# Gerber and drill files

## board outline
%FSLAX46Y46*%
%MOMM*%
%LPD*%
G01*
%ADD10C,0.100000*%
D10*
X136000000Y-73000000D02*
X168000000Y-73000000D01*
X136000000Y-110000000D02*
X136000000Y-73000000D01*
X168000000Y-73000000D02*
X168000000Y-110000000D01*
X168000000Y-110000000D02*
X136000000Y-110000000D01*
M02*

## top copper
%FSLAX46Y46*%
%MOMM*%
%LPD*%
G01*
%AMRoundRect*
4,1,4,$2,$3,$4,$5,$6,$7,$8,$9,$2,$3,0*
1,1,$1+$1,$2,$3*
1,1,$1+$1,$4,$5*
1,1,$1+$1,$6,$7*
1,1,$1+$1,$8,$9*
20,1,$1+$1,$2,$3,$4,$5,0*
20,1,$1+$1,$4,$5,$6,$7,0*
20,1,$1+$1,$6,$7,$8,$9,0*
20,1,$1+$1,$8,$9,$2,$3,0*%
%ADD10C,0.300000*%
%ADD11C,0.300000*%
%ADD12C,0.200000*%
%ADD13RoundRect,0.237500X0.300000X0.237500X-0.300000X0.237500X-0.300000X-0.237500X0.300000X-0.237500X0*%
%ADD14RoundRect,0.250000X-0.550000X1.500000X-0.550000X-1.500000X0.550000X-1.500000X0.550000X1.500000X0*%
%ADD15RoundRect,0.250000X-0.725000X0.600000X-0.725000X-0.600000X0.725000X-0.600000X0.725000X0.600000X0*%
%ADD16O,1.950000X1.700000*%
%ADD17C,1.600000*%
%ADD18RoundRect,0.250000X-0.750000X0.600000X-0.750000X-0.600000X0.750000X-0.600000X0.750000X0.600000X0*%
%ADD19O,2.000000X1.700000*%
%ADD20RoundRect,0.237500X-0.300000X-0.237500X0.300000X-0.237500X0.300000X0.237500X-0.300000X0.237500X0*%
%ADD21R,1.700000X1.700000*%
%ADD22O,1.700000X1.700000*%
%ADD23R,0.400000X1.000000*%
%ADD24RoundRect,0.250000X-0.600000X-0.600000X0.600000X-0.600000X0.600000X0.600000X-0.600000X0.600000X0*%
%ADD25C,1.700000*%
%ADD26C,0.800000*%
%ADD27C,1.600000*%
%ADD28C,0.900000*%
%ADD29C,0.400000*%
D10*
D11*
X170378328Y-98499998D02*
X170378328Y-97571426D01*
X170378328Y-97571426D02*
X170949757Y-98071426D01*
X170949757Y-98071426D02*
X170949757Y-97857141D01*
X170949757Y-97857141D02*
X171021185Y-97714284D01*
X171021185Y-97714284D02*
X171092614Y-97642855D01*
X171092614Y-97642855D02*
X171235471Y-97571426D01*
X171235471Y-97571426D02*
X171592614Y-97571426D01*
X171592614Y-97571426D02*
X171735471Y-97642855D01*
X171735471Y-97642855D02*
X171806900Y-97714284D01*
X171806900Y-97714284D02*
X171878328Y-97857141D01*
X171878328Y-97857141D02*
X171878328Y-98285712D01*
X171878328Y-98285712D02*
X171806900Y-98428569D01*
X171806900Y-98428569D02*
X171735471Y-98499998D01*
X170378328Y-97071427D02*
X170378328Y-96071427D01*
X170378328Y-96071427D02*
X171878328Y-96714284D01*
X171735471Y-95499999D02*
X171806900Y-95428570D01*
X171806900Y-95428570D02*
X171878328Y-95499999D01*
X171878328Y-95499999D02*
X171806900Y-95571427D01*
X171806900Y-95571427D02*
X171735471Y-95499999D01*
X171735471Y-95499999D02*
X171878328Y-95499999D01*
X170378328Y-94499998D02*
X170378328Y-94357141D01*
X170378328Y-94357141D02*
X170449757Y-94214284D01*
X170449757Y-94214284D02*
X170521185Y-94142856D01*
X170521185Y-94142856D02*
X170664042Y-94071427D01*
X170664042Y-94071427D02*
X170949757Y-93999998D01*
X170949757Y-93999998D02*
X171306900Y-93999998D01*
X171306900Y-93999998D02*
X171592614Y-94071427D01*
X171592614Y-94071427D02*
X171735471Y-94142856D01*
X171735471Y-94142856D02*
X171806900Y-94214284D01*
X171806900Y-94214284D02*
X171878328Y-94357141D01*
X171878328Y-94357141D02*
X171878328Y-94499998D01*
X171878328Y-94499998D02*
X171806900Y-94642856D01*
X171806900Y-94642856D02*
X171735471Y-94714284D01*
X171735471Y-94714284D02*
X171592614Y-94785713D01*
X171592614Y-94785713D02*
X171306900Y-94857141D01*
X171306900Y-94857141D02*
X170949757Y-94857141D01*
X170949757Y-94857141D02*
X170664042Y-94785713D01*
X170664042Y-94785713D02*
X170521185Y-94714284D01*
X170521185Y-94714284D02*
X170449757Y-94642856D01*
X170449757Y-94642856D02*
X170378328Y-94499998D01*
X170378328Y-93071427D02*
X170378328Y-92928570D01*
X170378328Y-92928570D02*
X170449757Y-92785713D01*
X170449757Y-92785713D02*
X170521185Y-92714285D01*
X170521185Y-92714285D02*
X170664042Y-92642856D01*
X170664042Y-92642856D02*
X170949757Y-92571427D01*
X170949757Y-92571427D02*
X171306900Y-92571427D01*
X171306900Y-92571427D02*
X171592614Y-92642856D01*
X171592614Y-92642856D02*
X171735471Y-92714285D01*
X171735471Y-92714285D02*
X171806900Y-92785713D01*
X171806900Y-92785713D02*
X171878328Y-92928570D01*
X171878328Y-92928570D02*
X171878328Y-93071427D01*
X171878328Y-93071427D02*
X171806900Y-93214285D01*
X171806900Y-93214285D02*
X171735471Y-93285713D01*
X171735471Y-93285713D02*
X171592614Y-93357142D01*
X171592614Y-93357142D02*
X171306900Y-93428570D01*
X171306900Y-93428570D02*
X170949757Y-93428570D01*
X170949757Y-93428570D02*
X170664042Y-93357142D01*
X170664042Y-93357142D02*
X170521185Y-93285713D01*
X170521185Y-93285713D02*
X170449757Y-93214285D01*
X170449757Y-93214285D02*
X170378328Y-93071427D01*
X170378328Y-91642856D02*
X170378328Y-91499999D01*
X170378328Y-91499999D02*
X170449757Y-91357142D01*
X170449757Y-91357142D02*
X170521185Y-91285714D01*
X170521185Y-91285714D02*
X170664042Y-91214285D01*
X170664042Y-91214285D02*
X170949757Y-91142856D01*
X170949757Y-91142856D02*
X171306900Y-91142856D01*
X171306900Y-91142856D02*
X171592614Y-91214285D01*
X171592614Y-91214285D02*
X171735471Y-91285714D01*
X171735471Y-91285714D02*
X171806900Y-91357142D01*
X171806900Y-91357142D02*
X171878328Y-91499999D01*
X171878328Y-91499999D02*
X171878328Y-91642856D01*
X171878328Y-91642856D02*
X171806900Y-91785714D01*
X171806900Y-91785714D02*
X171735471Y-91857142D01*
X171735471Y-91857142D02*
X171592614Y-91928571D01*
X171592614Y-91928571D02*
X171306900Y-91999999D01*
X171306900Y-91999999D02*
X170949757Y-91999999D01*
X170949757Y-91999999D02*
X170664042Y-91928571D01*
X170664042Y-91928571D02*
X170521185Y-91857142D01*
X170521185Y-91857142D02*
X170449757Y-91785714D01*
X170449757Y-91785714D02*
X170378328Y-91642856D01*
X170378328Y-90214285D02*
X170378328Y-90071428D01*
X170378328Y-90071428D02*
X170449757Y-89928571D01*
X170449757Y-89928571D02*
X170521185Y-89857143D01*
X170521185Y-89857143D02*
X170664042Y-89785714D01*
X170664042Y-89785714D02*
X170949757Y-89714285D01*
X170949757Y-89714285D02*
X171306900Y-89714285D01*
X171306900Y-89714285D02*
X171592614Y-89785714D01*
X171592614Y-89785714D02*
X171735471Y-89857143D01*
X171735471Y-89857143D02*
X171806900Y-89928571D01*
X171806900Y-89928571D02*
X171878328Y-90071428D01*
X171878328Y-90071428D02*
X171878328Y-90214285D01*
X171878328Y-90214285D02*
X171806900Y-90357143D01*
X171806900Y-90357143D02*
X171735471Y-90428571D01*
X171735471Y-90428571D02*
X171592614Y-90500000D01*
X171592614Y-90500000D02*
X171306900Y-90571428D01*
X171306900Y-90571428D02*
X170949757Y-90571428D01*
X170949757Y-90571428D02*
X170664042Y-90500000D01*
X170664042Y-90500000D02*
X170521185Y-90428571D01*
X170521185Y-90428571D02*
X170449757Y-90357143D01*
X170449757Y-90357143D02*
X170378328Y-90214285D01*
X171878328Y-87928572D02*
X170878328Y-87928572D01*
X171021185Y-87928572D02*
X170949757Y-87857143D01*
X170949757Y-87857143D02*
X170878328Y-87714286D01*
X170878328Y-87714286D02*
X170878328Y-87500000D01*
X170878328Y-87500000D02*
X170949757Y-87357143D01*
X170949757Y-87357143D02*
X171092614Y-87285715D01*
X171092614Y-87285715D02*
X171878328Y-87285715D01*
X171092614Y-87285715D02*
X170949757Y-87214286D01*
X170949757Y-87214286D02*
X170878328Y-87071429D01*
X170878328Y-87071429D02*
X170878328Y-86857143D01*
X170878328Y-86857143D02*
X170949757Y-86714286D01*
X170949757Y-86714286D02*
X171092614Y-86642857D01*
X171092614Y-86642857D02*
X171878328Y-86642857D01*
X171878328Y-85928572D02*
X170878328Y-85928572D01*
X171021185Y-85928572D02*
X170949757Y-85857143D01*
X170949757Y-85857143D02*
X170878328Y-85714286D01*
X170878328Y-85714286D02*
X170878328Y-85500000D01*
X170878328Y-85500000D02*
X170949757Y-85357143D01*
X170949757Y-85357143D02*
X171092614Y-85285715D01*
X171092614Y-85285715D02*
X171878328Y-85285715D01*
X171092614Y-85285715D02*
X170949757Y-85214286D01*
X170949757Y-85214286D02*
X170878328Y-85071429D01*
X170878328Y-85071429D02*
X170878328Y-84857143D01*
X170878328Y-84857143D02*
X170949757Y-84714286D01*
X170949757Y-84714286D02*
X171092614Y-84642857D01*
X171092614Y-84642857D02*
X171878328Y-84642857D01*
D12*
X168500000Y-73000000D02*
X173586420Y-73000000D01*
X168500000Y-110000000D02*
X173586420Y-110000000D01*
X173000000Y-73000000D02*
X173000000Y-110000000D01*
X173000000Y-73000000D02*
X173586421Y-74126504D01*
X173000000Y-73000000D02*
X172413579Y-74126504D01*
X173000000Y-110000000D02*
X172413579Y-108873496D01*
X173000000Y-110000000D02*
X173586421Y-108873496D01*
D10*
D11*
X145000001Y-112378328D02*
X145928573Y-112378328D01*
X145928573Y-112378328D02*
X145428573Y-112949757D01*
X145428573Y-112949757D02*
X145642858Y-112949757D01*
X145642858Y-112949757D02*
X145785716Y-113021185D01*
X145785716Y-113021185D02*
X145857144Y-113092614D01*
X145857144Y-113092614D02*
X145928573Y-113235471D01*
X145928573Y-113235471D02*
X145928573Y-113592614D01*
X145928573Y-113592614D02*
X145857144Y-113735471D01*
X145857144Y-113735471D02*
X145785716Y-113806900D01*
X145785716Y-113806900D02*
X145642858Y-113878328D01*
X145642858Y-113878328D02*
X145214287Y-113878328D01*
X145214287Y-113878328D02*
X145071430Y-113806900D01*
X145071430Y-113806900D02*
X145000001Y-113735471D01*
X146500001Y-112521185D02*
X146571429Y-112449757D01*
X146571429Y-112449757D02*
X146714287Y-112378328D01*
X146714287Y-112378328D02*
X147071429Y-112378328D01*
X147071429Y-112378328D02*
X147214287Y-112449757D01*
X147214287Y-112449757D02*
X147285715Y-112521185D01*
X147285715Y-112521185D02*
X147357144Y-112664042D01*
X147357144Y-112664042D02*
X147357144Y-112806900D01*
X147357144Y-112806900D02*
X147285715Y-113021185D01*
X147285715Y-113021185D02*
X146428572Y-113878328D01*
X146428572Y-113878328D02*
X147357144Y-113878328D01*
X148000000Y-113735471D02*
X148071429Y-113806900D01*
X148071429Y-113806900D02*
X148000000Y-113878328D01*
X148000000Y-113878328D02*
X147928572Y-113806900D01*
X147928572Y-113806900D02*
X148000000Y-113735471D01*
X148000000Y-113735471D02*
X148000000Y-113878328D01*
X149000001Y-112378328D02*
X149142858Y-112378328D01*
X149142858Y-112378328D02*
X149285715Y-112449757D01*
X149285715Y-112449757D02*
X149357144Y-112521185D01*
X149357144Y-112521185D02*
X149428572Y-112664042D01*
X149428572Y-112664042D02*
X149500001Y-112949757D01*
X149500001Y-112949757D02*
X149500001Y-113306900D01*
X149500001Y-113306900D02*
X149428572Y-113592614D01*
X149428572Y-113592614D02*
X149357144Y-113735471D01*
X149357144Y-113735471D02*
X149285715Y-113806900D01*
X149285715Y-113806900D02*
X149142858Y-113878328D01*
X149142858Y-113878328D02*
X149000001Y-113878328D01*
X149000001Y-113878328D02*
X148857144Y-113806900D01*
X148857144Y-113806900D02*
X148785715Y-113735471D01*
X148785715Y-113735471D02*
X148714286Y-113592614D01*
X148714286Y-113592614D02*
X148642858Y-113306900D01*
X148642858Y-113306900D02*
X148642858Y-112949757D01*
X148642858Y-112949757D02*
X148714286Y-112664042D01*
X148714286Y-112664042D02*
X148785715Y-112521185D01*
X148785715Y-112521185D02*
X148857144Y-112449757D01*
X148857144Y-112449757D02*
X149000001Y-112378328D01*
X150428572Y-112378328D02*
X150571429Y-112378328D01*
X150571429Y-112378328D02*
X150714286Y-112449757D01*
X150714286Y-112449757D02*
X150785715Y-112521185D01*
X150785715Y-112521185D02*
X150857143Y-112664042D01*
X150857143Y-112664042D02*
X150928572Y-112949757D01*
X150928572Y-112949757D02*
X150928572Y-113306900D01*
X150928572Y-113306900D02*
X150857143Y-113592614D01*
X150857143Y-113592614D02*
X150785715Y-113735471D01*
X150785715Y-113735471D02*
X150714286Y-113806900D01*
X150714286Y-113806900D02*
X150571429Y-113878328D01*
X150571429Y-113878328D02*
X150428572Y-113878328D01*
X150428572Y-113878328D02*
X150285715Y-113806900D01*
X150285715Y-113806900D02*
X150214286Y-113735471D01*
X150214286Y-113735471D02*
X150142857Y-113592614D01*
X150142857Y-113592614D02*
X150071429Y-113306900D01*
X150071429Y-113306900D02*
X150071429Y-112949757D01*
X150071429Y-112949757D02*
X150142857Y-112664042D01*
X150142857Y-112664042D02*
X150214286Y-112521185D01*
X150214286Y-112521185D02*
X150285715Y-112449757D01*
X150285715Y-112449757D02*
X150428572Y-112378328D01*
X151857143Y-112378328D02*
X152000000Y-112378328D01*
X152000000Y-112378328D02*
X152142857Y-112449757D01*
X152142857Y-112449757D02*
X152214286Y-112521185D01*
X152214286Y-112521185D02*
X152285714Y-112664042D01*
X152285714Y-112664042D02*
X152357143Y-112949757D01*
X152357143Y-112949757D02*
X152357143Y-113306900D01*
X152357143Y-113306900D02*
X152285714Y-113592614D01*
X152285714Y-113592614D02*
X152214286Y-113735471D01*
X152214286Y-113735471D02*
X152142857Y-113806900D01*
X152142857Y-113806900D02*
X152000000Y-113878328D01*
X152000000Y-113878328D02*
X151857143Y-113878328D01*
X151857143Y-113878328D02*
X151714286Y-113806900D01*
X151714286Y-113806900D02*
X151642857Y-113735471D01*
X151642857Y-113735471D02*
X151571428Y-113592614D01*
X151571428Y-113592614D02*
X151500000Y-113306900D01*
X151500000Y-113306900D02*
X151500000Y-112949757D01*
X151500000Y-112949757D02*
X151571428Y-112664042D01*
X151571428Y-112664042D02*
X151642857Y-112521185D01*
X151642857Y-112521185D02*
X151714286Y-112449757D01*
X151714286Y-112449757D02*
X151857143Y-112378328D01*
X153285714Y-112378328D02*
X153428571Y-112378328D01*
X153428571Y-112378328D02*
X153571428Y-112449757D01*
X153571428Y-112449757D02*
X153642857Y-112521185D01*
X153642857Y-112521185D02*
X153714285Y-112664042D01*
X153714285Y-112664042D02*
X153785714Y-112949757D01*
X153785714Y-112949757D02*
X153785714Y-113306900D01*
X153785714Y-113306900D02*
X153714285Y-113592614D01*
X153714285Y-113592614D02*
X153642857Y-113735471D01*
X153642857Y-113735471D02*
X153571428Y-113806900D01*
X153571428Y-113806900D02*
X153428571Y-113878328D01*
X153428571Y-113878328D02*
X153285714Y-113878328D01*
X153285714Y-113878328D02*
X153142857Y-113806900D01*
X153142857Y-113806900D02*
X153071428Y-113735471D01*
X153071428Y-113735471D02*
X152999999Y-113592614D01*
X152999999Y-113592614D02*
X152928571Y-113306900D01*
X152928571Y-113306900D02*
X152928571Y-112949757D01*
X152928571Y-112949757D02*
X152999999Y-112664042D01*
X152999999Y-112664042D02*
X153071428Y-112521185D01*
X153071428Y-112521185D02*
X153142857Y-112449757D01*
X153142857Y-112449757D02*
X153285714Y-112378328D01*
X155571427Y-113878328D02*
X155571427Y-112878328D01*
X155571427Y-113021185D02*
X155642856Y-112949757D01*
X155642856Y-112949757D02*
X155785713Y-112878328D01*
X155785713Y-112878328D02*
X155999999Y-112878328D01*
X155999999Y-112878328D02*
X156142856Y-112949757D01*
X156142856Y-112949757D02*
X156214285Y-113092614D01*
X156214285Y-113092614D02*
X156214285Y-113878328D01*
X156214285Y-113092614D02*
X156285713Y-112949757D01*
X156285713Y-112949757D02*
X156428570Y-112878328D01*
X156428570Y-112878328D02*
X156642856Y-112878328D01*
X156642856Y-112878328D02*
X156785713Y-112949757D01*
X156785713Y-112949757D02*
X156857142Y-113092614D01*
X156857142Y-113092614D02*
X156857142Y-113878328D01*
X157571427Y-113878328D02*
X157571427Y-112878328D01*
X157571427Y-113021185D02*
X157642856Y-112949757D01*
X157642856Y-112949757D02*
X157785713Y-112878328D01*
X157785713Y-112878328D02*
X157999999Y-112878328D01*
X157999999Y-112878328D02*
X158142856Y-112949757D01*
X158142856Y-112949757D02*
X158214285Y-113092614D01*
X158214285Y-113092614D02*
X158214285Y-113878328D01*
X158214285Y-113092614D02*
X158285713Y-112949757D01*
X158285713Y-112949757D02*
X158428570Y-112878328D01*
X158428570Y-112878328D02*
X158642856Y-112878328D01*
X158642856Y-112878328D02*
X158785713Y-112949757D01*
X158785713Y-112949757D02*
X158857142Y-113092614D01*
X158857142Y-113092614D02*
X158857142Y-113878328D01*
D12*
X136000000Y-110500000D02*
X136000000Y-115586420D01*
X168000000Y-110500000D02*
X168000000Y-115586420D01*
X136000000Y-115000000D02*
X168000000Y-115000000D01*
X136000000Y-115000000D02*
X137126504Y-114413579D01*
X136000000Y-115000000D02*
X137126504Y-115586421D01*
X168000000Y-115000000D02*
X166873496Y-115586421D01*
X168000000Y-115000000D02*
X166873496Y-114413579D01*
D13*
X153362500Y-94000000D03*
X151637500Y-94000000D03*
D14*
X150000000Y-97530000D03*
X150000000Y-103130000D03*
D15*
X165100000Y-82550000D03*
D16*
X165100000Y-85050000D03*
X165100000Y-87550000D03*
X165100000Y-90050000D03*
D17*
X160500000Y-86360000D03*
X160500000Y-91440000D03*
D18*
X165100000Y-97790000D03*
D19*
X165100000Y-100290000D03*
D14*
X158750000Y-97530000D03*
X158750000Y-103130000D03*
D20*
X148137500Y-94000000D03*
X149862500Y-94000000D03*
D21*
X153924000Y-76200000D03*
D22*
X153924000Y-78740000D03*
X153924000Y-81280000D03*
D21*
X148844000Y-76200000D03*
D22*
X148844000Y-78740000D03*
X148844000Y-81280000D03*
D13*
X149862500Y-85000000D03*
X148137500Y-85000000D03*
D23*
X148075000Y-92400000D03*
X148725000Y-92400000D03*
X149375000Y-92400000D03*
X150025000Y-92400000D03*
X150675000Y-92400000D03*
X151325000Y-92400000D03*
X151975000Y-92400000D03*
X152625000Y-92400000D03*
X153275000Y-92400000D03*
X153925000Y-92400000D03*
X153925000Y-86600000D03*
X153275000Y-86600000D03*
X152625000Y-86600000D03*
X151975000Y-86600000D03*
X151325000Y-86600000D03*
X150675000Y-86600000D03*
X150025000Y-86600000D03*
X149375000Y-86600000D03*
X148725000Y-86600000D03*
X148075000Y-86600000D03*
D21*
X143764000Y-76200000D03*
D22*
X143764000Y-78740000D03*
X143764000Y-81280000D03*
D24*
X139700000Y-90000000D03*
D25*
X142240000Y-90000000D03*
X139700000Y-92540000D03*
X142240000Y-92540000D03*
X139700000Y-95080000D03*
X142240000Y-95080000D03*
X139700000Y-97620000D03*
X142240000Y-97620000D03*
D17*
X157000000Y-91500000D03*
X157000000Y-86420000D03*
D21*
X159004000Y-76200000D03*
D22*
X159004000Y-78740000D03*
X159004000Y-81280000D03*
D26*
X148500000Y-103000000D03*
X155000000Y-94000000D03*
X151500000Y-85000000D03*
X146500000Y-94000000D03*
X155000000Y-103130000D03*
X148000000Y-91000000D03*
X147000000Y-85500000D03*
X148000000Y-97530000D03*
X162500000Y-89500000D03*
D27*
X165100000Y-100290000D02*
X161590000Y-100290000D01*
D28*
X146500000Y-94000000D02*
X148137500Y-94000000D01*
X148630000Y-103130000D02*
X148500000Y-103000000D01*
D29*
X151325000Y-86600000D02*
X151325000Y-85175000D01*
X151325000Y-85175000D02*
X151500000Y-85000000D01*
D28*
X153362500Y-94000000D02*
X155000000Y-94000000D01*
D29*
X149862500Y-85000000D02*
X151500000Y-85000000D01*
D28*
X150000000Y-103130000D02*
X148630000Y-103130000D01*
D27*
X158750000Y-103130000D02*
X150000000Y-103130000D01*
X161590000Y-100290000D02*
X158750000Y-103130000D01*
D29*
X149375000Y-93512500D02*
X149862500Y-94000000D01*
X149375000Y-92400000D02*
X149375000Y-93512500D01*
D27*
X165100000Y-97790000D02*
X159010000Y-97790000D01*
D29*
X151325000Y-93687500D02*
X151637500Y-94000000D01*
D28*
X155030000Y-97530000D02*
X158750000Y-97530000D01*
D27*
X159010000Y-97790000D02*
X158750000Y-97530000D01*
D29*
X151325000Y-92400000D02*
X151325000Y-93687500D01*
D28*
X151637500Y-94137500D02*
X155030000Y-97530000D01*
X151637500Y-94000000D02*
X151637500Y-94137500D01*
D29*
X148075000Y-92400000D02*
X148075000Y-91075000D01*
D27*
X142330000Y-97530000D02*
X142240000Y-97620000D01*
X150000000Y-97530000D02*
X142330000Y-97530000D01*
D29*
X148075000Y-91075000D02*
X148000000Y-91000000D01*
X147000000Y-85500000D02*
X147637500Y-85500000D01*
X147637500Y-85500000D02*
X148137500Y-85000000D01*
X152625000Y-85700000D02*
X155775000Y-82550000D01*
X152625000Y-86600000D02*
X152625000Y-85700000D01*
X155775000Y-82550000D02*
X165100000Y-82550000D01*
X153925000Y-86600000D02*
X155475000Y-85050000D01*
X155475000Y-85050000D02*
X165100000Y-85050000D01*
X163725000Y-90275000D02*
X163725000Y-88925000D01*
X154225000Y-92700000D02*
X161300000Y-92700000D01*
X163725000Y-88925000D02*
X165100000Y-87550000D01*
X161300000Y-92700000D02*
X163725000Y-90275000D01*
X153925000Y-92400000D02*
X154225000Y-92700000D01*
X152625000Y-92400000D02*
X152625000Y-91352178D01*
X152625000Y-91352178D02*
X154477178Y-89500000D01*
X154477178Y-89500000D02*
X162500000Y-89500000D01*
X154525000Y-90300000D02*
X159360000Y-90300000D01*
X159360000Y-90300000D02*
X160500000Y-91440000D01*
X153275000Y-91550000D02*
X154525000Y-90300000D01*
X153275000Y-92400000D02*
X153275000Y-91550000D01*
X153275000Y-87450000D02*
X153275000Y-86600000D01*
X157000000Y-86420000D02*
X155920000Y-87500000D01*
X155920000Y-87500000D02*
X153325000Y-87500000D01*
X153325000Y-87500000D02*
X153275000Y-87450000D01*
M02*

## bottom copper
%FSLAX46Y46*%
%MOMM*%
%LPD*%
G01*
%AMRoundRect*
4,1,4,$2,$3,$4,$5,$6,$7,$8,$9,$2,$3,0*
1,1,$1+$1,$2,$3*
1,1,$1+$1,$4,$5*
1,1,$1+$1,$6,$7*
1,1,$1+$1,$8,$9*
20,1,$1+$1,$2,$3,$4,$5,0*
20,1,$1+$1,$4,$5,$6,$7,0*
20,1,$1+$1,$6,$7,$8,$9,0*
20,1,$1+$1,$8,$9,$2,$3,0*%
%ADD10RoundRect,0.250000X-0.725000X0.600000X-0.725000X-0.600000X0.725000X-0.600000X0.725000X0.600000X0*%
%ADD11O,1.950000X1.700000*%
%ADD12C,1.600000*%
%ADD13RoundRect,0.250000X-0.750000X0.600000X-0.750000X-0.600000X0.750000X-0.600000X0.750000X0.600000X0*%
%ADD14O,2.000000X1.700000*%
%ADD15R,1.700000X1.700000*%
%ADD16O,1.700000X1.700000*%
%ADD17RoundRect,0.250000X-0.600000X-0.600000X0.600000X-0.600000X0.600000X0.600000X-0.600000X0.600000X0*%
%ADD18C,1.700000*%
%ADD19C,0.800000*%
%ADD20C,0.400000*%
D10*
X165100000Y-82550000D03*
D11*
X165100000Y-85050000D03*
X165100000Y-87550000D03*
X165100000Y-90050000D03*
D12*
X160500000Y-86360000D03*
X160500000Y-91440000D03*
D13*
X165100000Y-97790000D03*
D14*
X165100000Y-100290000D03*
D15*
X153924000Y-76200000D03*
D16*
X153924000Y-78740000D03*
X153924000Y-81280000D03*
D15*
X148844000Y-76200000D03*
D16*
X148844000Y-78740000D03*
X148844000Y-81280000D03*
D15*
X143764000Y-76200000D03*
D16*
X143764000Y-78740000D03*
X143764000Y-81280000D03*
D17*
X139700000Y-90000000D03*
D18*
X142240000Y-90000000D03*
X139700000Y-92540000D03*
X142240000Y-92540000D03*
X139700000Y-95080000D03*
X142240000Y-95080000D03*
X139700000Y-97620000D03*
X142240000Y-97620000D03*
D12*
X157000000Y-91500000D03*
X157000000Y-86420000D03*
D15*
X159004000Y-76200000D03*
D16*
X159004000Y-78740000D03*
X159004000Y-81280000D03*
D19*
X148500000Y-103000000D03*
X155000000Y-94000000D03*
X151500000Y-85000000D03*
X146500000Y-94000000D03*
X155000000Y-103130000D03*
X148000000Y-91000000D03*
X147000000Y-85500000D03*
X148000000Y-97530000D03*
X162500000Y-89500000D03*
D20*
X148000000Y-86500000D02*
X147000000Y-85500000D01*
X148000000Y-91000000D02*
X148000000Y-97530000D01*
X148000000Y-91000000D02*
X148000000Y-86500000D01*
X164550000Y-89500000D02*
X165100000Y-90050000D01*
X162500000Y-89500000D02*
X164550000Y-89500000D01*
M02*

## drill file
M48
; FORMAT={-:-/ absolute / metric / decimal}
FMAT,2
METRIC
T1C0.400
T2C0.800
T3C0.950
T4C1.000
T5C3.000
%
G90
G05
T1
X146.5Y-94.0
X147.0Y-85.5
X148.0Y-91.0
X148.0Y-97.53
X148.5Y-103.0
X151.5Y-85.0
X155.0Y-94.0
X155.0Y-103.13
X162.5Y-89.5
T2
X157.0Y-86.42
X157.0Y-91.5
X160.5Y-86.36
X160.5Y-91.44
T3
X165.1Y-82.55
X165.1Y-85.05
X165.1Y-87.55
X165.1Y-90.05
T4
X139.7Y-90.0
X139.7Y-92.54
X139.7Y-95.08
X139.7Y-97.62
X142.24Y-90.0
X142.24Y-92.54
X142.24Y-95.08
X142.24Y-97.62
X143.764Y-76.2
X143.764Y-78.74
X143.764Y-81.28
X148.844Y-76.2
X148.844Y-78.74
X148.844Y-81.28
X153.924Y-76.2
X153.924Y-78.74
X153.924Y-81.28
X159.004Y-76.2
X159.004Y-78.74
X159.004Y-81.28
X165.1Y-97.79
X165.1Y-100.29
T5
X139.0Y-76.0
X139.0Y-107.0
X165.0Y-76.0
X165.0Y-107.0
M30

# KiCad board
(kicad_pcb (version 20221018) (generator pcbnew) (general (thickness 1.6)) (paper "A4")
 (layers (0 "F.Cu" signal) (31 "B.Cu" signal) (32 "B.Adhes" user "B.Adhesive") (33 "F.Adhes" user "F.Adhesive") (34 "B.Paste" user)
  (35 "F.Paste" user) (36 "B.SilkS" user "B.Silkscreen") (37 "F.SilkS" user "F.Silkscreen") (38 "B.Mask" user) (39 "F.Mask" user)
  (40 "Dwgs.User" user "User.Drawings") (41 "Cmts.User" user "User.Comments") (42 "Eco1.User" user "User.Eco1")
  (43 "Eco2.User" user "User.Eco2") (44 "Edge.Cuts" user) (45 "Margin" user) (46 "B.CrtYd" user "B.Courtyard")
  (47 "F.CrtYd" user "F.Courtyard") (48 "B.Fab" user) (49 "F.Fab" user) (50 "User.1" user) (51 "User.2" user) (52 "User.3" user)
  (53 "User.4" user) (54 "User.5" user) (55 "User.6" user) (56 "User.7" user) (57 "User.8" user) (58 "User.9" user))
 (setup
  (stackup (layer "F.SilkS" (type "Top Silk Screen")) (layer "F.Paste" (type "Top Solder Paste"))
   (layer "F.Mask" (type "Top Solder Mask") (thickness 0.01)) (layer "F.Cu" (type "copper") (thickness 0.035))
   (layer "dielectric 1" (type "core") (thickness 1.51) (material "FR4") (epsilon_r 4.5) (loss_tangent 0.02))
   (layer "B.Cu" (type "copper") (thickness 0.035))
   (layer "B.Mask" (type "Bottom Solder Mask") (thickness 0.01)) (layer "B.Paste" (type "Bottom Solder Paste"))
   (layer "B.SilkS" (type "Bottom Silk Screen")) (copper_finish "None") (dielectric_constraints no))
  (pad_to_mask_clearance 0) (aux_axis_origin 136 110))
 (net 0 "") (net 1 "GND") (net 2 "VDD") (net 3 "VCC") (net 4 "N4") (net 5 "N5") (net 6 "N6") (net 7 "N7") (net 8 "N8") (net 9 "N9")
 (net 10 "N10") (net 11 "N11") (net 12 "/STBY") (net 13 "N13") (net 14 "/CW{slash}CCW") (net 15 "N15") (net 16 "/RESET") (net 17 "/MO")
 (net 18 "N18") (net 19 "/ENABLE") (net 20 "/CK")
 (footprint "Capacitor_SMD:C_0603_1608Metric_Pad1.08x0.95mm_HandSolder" (layer "F.Cu") (at 152.5 94 180)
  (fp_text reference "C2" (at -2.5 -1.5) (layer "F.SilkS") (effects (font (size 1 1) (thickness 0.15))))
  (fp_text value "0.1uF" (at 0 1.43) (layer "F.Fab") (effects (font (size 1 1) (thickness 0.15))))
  (pad "1" smd roundrect (at -0.8625 0 180) (size 1.075 0.95) (layers "F.Cu" "F.Paste" "F.Mask") (roundrect_rratio 0.25) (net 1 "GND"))
  (pad "2" smd roundrect (at 0.8625 0 180) (size 1.075 0.95) (layers "F.Cu" "F.Paste" "F.Mask") (roundrect_rratio 0.25) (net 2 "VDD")))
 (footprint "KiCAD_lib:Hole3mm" (layer "F.Cu") (at 165 107)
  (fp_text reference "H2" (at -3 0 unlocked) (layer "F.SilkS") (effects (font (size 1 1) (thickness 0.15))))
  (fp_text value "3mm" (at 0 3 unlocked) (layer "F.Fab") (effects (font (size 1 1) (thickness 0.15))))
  (pad "" np_thru_hole circle (at 0 0) (size 3 3) (drill 3) (layers "F&B.Cu")))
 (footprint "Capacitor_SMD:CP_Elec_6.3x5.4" (layer "F.Cu") (at 150 100.33 -90)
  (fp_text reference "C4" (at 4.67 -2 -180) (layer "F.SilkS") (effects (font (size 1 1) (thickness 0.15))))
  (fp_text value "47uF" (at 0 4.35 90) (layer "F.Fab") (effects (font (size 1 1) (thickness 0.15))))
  (pad "1" smd roundrect (at -2.8 0 270) (size 3.5 1.6) (layers "F.Cu" "F.Paste" "F.Mask") (roundrect_rratio 0.15625) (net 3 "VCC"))
  (pad "2" smd roundrect (at 2.8 0 270) (size 3.5 1.6) (layers "F.Cu" "F.Paste" "F.Mask") (roundrect_rratio 0.15625) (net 1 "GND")))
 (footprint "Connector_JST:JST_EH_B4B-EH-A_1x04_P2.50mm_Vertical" (layer "F.Cu") (at 165.1 82.55 -90)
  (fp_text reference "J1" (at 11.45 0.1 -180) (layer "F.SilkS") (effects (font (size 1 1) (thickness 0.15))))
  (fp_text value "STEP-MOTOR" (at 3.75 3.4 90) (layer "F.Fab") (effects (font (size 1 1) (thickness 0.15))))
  (pad "1" thru_hole roundrect (at 0 0 270) (size 1.7 1.95) (drill 0.95) (layers "*.Cu" "*.Mask") (roundrect_rratio 0.147059) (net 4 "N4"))
  (pad "2" thru_hole oval (at 2.5 0 270) (size 1.7 1.95) (drill 0.95) (layers "*.Cu" "*.Mask") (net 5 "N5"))
  (pad "3" thru_hole oval (at 5 0 270) (size 1.7 1.95) (drill 0.95) (layers "*.Cu" "*.Mask") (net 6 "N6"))
  (pad "4" thru_hole oval (at 7.5 0 270) (size 1.7 1.95) (drill 0.95) (layers "*.Cu" "*.Mask") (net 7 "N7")))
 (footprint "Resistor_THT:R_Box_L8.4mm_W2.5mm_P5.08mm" (layer "F.Cu") (at 160.5 86.36 -90)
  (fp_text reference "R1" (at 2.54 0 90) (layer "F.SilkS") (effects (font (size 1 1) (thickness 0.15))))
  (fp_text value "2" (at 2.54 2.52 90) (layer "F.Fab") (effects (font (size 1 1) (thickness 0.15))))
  (pad "1" thru_hole circle (at 0 0 270) (size 1.6 1.6) (drill 0.8) (layers "*.Cu" "*.Mask") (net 1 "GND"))
  (pad "2" thru_hole circle (at 5.08 0 270) (size 1.6 1.6) (drill 0.8) (layers "*.Cu" "*.Mask") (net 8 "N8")))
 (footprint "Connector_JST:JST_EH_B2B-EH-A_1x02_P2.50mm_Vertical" (layer "F.Cu") (at 165.1 97.79 -90)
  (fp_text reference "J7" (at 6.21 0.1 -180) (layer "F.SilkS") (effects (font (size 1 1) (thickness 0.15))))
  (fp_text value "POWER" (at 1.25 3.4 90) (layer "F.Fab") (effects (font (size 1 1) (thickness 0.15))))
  (pad "1" thru_hole roundrect (at 0 0 270) (size 1.7 2) (drill 1) (layers "*.Cu" "*.Mask") (roundrect_rratio 0.147059) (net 2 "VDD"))
  (pad "2" thru_hole oval (at 2.5 0 270) (size 1.7 2) (drill 1) (layers "*.Cu" "*.Mask") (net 1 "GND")))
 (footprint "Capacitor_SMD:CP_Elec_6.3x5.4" (layer "F.Cu") (at 158.75 100.33 -90)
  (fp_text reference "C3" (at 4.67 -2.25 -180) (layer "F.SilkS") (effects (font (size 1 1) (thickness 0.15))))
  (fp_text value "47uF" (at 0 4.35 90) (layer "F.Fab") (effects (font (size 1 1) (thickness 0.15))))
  (pad "1" smd roundrect (at -2.8 0 270) (size 3.5 1.6) (layers "F.Cu" "F.Paste" "F.Mask") (roundrect_rratio 0.15625) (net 2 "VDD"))
  (pad "2" smd roundrect (at 2.8 0 270) (size 3.5 1.6) (layers "F.Cu" "F.Paste" "F.Mask") (roundrect_rratio 0.15625) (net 1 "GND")))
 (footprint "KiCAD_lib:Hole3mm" (layer "F.Cu") (at 139 107)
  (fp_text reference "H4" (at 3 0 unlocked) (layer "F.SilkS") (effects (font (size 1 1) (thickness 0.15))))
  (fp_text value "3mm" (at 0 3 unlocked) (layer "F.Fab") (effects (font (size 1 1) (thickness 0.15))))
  (pad "" np_thru_hole circle (at 0 0) (size 3 3) (drill 3) (layers "F&B.Cu")))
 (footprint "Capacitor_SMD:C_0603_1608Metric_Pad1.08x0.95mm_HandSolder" (layer "F.Cu") (at 149 94)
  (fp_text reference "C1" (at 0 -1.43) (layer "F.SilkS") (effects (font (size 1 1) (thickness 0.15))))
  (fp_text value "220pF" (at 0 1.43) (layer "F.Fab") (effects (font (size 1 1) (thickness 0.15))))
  (pad "1" smd roundrect (at -0.8625 0) (size 1.075 0.95) (layers "F.Cu" "F.Paste" "F.Mask") (roundrect_rratio 0.25) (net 1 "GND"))
  (pad "2" smd roundrect (at 0.8625 0) (size 1.075 0.95) (layers "F.Cu" "F.Paste" "F.Mask") (roundrect_rratio 0.25) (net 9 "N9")))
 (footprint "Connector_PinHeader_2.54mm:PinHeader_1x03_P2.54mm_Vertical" (layer "F.Cu") (at 153.924 76.2)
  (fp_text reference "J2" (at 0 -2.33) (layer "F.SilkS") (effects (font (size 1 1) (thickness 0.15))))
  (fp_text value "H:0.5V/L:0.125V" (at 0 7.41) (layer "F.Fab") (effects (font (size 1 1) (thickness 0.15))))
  (pad "1" thru_hole rect (at 0 0) (size 1.7 1.7) (drill 1) (layers "*.Cu" "*.Mask") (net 3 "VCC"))
  (pad "2" thru_hole oval (at 0 2.54) (size 1.7 1.7) (drill 1) (layers "*.Cu" "*.Mask") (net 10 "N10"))
  (pad "3" thru_hole oval (at 0 5.08) (size 1.7 1.7) (drill 1) (layers "*.Cu" "*.Mask") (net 1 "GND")))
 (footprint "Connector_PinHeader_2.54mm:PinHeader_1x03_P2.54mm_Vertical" (layer "F.Cu") (at 148.844 76.2)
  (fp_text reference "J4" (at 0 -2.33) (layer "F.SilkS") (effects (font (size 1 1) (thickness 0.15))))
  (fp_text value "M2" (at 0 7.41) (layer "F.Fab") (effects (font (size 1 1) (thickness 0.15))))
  (pad "1" thru_hole rect (at 0 0) (size 1.7 1.7) (drill 1) (layers "*.Cu" "*.Mask") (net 3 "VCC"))
  (pad "2" thru_hole oval (at 0 2.54) (size 1.7 1.7) (drill 1) (layers "*.Cu" "*.Mask") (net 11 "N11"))
  (pad "3" thru_hole oval (at 0 5.08) (size 1.7 1.7) (drill 1) (layers "*.Cu" "*.Mask") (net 1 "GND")))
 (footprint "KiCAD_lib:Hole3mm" (layer "F.Cu") (at 139 76)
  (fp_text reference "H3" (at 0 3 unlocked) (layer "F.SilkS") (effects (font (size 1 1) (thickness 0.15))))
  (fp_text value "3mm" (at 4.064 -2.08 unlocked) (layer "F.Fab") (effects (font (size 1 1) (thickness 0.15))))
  (pad "" np_thru_hole circle (at 0 0) (size 3 3) (drill 3) (layers "F&B.Cu")))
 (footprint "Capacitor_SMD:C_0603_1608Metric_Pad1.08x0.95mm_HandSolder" (layer "F.Cu") (at 149 85 180)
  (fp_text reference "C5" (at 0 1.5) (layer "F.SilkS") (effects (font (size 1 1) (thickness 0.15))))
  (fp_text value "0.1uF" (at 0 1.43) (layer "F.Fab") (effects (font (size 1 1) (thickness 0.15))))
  (pad "1" smd roundrect (at -0.8625 0 180) (size 1.075 0.95) (layers "F.Cu" "F.Paste" "F.Mask") (roundrect_rratio 0.25) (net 1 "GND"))
  (pad "2" smd roundrect (at 0.8625 0 180) (size 1.075 0.95) (layers "F.Cu" "F.Paste" "F.Mask") (roundrect_rratio 0.25) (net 3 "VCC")))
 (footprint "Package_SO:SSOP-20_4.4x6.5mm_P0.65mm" (layer "F.Cu") (at 151 89.5 90)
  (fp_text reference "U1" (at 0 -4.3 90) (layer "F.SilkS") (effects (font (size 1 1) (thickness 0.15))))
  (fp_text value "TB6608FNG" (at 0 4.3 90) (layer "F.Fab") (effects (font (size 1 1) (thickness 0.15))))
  (pad "1" smd rect (at -2.9 -2.925 90) (size 1 0.4) (layers "F.Cu" "F.Paste" "F.Mask") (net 3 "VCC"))
  (pad "2" smd rect (at -2.9 -2.275 90) (size 1 0.4) (layers "F.Cu" "F.Paste" "F.Mask") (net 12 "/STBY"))
  (pad "3" smd rect (at -2.9 -1.625 90) (size 1 0.4) (layers "F.Cu" "F.Paste" "F.Mask") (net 9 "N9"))
  (pad "4" smd rect (at -2.9 -0.975 90) (size 1 0.4) (layers "F.Cu" "F.Paste" "F.Mask") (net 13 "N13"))
  (pad "5" smd rect (at -2.9 -0.325 90) (size 1 0.4) (layers "F.Cu" "F.Paste" "F.Mask") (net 11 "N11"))
  (pad "6" smd rect (at -2.9 0.325 90) (size 1 0.4) (layers "F.Cu" "F.Paste" "F.Mask") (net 2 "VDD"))
  (pad "7" smd rect (at -2.9 0.975 90) (size 1 0.4) (layers "F.Cu" "F.Paste" "F.Mask") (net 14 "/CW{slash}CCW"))
  (pad "8" smd rect (at -2.9 1.625 90) (size 1 0.4) (layers "F.Cu" "F.Paste" "F.Mask") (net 7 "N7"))
  (pad "9" smd rect (at -2.9 2.275 90) (size 1 0.4) (layers "F.Cu" "F.Paste" "F.Mask") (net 8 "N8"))
  (pad "10" smd rect (at -2.9 2.925 90) (size 1 0.4) (layers "F.Cu" "F.Paste" "F.Mask") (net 6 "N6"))
  (pad "11" smd rect (at 2.9 2.925 90) (size 1 0.4) (layers "F.Cu" "F.Paste" "F.Mask") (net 5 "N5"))
  (pad "12" smd rect (at 2.9 2.275 90) (size 1 0.4) (layers "F.Cu" "F.Paste" "F.Mask") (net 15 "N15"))
  (pad "13" smd rect (at 2.9 1.625 90) (size 1 0.4) (layers "F.Cu" "F.Paste" "F.Mask") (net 4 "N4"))
  (pad "14" smd rect (at 2.9 0.975 90) (size 1 0.4) (layers "F.Cu" "F.Paste" "F.Mask") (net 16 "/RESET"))
  (pad "15" smd rect (at 2.9 0.325 90) (size 1 0.4) (layers "F.Cu" "F.Paste" "F.Mask") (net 1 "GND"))
  (pad "16" smd rect (at 2.9 -0.325 90) (size 1 0.4) (layers "F.Cu" "F.Paste" "F.Mask") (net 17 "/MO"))
  (pad "17" smd rect (at 2.9 -0.975 90) (size 1 0.4) (layers "F.Cu" "F.Paste" "F.Mask") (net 10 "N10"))
  (pad "18" smd rect (at 2.9 -1.625 90) (size 1 0.4) (layers "F.Cu" "F.Paste" "F.Mask") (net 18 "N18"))
  (pad "19" smd rect (at 2.9 -2.275 90) (size 1 0.4) (layers "F.Cu" "F.Paste" "F.Mask") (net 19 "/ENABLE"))
  (pad "20" smd rect (at 2.9 -2.925 90) (size 1 0.4) (layers "F.Cu" "F.Paste" "F.Mask") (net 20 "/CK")))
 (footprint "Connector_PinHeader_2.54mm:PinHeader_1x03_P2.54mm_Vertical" (layer "F.Cu") (at 143.764 76.2)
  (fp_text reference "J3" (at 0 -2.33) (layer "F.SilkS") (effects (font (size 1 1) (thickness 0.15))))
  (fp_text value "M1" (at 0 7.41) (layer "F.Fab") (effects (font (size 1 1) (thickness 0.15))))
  (pad "1" thru_hole rect (at 0 0) (size 1.7 1.7) (drill 1) (layers "*.Cu" "*.Mask") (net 3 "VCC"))
  (pad "2" thru_hole oval (at 0 2.54) (size 1.7 1.7) (drill 1) (layers "*.Cu" "*.Mask") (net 13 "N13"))
  (pad "3" thru_hole oval (at 0 5.08) (size 1.7 1.7) (drill 1) (layers "*.Cu" "*.Mask") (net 1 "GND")))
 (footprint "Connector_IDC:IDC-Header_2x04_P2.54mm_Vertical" (layer "F.Cu") (at 139.7 90)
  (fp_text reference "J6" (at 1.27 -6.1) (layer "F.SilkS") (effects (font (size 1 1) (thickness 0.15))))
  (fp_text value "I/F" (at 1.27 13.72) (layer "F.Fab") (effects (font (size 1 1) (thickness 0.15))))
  (pad "1" thru_hole roundrect (at 0 0) (size 1.7 1.7) (drill 1) (layers "*.Cu" "*.Mask") (roundrect_rratio 0.147059)
   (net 14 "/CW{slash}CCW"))
  (pad "2" thru_hole circle (at 2.54 0) (size 1.7 1.7) (drill 1) (layers "*.Cu" "*.Mask") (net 20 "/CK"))
  (pad "3" thru_hole circle (at 0 2.54) (size 1.7 1.7) (drill 1) (layers "*.Cu" "*.Mask") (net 16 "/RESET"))
  (pad "4" thru_hole circle (at 2.54 2.54) (size 1.7 1.7) (drill 1) (layers "*.Cu" "*.Mask") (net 19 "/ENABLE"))
  (pad "5" thru_hole circle (at 0 5.08) (size 1.7 1.7) (drill 1) (layers "*.Cu" "*.Mask") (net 12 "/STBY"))
  (pad "6" thru_hole circle (at 2.54 5.08) (size 1.7 1.7) (drill 1) (layers "*.Cu" "*.Mask") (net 17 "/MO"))
  (pad "7" thru_hole circle (at 0 7.62) (size 1.7 1.7) (drill 1) (layers "*.Cu" "*.Mask") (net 1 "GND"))
  (pad "8" thru_hole circle (at 2.54 7.62) (size 1.7 1.7) (drill 1) (layers "*.Cu" "*.Mask") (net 3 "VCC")))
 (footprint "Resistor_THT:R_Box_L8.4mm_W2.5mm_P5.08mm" (layer "F.Cu") (at 157 91.5 90)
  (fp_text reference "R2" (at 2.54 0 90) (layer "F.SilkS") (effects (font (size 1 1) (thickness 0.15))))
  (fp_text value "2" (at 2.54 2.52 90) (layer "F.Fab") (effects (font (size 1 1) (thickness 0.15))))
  (pad "1" thru_hole circle (at 0 0 90) (size 1.6 1.6) (drill 0.8) (layers "*.Cu" "*.Mask") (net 1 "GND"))
  (pad "2" thru_hole circle (at 5.08 0 90) (size 1.6 1.6) (drill 0.8) (layers "*.Cu" "*.Mask") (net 15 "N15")))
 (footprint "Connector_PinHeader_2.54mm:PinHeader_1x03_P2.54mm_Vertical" (layer "F.Cu") (at 159.004 76.2)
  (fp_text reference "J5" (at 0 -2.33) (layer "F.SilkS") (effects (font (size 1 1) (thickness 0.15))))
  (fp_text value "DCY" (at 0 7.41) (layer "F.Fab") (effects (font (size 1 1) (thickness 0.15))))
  (pad "1" thru_hole rect (at 0 0) (size 1.7 1.7) (drill 1) (layers "*.Cu" "*.Mask") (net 3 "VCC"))
  (pad "2" thru_hole oval (at 0 2.54) (size 1.7 1.7) (drill 1) (layers "*.Cu" "*.Mask") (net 18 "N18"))
  (pad "3" thru_hole oval (at 0 5.08) (size 1.7 1.7) (drill 1) (layers "*.Cu" "*.Mask") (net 1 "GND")))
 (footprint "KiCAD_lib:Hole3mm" (layer "F.Cu") (at 165 76)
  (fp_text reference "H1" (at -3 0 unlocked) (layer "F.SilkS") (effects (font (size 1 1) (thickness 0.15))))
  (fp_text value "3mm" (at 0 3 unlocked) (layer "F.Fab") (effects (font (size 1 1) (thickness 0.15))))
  (pad "" np_thru_hole circle (at 0 0) (size 3 3) (drill 3) (layers "F&B.Cu")))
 (gr_line (start 136 73) (end 168 73) (stroke (width 0.1) (type default)) (layer "Edge.Cuts"))
 (gr_line (start 136 110) (end 136 73) (stroke (width 0.1) (type default)) (layer "Edge.Cuts"))
 (gr_line (start 168 73) (end 168 110) (stroke (width 0.1) (type default)) (layer "Edge.Cuts"))
 (gr_line (start 168 110) (end 136 110) (stroke (width 0.1) (type default)) (layer "Edge.Cuts"))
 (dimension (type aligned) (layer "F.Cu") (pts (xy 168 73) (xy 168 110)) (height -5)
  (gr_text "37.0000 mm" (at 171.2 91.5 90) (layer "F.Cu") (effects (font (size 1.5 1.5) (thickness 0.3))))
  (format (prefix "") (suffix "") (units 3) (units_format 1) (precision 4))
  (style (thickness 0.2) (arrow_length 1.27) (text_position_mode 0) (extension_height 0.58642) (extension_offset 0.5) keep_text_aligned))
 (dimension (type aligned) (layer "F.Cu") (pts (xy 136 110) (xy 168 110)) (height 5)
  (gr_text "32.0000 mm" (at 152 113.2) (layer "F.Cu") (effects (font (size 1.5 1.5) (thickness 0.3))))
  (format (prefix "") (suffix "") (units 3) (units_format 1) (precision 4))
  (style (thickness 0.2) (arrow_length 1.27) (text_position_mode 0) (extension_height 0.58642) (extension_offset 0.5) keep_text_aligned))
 (segment (start 165.1 100.29) (end 161.59 100.29) (width 1.6) (layer "F.Cu") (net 1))
 (segment (start 146.5 94) (end 148.1375 94) (width 0.9) (layer "F.Cu") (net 1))
 (segment (start 148.63 103.13) (end 148.5 103) (width 0.9) (layer "F.Cu") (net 1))
 (segment (start 151.325 86.6) (end 151.325 85.175) (width 0.4) (layer "F.Cu") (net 1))
 (segment (start 151.325 85.175) (end 151.5 85) (width 0.4) (layer "F.Cu") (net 1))
 (segment (start 153.3625 94) (end 155 94) (width 0.9) (layer "F.Cu") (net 1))
 (segment (start 149.8625 85) (end 151.5 85) (width 0.4) (layer "F.Cu") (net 1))
 (segment (start 150 103.13) (end 148.63 103.13) (width 0.9) (layer "F.Cu") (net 1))
 (segment (start 158.75 103.13) (end 150 103.13) (width 1.6) (layer "F.Cu") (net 1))
 (segment (start 161.59 100.29) (end 158.75 103.13) (width 1.6) (layer "F.Cu") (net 1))
 (via (at 148.5 103) (size 0.8) (drill 0.4) (layers "F.Cu" "B.Cu") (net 1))
 (via (at 155 94) (size 0.8) (drill 0.4) (layers "F.Cu" "B.Cu") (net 1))
 (via (at 151.5 85) (size 0.8) (drill 0.4) (layers "F.Cu" "B.Cu") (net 1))
 (via (at 146.5 94) (size 0.8) (drill 0.4) (layers "F.Cu" "B.Cu") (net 1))
 (via (at 155 103.13) (size 0.8) (drill 0.4) (layers "F.Cu" "B.Cu") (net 1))
 (segment (start 149.375 93.5125) (end 149.8625 94) (width 0.4) (layer "F.Cu") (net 9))
 (segment (start 149.375 92.4) (end 149.375 93.5125) (width 0.4) (layer "F.Cu") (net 9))
 (segment (start 165.1 97.79) (end 159.01 97.79) (width 1.6) (layer "F.Cu") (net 2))
 (segment (start 151.325 93.6875) (end 151.6375 94) (width 0.4) (layer "F.Cu") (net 2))
 (segment (start 155.03 97.53) (end 158.75 97.53) (width 0.9) (layer "F.Cu") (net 2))
 (segment (start 159.01 97.79) (end 158.75 97.53) (width 1.6) (layer "F.Cu") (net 2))
 (segment (start 151.325 92.4) (end 151.325 93.6875) (width 0.4) (layer "F.Cu") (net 2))
 (segment (start 151.6375 94.1375) (end 155.03 97.53) (width 0.9) (layer "F.Cu") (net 2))
 (segment (start 151.6375 94) (end 151.6375 94.1375) (width 0.9) (layer "F.Cu") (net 2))
 (segment (start 148.075 92.4) (end 148.075 91.075) (width 0.4) (layer "F.Cu") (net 3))
 (segment (start 142.33 97.53) (end 142.24 97.62) (width 1.6) (layer "F.Cu") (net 3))
 (segment (start 150 97.53) (end 142.33 97.53) (width 1.6) (layer "F.Cu") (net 3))
 (segment (start 148.075 91.075) (end 148 91) (width 0.4) (layer "F.Cu") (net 3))
 (segment (start 147 85.5) (end 147.6375 85.5) (width 0.4) (layer "F.Cu") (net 3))
 (segment (start 147.6375 85.5) (end 148.1375 85) (width 0.4) (layer "F.Cu") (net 3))
 (via (at 148 91) (size 0.8) (drill 0.4) (layers "F.Cu" "B.Cu") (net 3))
 (via (at 147 85.5) (size 0.8) (drill 0.4) (layers "F.Cu" "B.Cu") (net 3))
 (via (at 148 97.53) (size 0.8) (drill 0.4) (layers "F.Cu" "B.Cu") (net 3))
 (segment (start 148 86.5) (end 147 85.5) (width 0.4) (layer "B.Cu") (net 3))
 (segment (start 148 91) (end 148 97.53) (width 0.4) (layer "B.Cu") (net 3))
 (segment (start 148 91) (end 148 86.5) (width 0.4) (layer "B.Cu") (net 3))
 (segment (start 152.625 85.7) (end 155.775 82.55) (width 0.4) (layer "F.Cu") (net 4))
 (segment (start 152.625 86.6) (end 152.625 85.7) (width 0.4) (layer "F.Cu") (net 4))
 (segment (start 155.775 82.55) (end 165.1 82.55) (width 0.4) (layer "F.Cu") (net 4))
 (segment (start 153.925 86.6) (end 155.475 85.05) (width 0.4) (layer "F.Cu") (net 5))
 (segment (start 155.475 85.05) (end 165.1 85.05) (width 0.4) (layer "F.Cu") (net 5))
 (segment (start 163.725 90.275) (end 163.725 88.925) (width 0.4) (layer "F.Cu") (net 6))
 (segment (start 154.225 92.7) (end 161.3 92.7) (width 0.4) (layer "F.Cu") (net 6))
 (segment (start 163.725 88.925) (end 165.1 87.55) (width 0.4) (layer "F.Cu") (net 6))
 (segment (start 161.3 92.7) (end 163.725 90.275) (width 0.4) (layer "F.Cu") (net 6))
 (segment (start 153.925 92.4) (end 154.225 92.7) (width 0.4) (layer "F.Cu") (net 6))
 (segment (start 152.625 92.4) (end 152.625 91.352178) (width 0.4) (layer "F.Cu") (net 7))
 (segment (start 152.625 91.352178) (end 154.477178 89.5) (width 0.4) (layer "F.Cu") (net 7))
 (segment (start 154.477178 89.5) (end 162.5 89.5) (width 0.4) (layer "F.Cu") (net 7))
 (via (at 162.5 89.5) (size 0.8) (drill 0.4) (layers "F.Cu" "B.Cu") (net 7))
 (segment (start 164.55 89.5) (end 165.1 90.05) (width 0.4) (layer "B.Cu") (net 7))
 (segment (start 162.5 89.5) (end 164.55 89.5) (width 0.4) (layer "B.Cu") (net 7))
 (segment (start 154.525 90.3) (end 159.36 90.3) (width 0.4) (layer "F.Cu") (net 8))
 (segment (start 159.36 90.3) (end 160.5 91.44) (width 0.4) (layer "F.Cu") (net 8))
 (segment (start 153.275 91.55) (end 154.525 90.3) (width 0.4) (layer "F.Cu") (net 8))
 (segment (start 153.275 92.4) (end 153.275 91.55) (width 0.4) (layer "F.Cu") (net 8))
 (segment (start 153.275 87.45) (end 153.275 86.6) (width 0.4) (layer "F.Cu") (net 15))
 (segment (start 157 86.42) (end 155.92 87.5) (width 0.4) (layer "F.Cu") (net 15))
 (segment (start 155.92 87.5) (end 153.325 87.5) (width 0.4) (layer "F.Cu") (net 15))
 (segment (start 153.325 87.5) (end 153.275 87.45) (width 0.4) (layer "F.Cu") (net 15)))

